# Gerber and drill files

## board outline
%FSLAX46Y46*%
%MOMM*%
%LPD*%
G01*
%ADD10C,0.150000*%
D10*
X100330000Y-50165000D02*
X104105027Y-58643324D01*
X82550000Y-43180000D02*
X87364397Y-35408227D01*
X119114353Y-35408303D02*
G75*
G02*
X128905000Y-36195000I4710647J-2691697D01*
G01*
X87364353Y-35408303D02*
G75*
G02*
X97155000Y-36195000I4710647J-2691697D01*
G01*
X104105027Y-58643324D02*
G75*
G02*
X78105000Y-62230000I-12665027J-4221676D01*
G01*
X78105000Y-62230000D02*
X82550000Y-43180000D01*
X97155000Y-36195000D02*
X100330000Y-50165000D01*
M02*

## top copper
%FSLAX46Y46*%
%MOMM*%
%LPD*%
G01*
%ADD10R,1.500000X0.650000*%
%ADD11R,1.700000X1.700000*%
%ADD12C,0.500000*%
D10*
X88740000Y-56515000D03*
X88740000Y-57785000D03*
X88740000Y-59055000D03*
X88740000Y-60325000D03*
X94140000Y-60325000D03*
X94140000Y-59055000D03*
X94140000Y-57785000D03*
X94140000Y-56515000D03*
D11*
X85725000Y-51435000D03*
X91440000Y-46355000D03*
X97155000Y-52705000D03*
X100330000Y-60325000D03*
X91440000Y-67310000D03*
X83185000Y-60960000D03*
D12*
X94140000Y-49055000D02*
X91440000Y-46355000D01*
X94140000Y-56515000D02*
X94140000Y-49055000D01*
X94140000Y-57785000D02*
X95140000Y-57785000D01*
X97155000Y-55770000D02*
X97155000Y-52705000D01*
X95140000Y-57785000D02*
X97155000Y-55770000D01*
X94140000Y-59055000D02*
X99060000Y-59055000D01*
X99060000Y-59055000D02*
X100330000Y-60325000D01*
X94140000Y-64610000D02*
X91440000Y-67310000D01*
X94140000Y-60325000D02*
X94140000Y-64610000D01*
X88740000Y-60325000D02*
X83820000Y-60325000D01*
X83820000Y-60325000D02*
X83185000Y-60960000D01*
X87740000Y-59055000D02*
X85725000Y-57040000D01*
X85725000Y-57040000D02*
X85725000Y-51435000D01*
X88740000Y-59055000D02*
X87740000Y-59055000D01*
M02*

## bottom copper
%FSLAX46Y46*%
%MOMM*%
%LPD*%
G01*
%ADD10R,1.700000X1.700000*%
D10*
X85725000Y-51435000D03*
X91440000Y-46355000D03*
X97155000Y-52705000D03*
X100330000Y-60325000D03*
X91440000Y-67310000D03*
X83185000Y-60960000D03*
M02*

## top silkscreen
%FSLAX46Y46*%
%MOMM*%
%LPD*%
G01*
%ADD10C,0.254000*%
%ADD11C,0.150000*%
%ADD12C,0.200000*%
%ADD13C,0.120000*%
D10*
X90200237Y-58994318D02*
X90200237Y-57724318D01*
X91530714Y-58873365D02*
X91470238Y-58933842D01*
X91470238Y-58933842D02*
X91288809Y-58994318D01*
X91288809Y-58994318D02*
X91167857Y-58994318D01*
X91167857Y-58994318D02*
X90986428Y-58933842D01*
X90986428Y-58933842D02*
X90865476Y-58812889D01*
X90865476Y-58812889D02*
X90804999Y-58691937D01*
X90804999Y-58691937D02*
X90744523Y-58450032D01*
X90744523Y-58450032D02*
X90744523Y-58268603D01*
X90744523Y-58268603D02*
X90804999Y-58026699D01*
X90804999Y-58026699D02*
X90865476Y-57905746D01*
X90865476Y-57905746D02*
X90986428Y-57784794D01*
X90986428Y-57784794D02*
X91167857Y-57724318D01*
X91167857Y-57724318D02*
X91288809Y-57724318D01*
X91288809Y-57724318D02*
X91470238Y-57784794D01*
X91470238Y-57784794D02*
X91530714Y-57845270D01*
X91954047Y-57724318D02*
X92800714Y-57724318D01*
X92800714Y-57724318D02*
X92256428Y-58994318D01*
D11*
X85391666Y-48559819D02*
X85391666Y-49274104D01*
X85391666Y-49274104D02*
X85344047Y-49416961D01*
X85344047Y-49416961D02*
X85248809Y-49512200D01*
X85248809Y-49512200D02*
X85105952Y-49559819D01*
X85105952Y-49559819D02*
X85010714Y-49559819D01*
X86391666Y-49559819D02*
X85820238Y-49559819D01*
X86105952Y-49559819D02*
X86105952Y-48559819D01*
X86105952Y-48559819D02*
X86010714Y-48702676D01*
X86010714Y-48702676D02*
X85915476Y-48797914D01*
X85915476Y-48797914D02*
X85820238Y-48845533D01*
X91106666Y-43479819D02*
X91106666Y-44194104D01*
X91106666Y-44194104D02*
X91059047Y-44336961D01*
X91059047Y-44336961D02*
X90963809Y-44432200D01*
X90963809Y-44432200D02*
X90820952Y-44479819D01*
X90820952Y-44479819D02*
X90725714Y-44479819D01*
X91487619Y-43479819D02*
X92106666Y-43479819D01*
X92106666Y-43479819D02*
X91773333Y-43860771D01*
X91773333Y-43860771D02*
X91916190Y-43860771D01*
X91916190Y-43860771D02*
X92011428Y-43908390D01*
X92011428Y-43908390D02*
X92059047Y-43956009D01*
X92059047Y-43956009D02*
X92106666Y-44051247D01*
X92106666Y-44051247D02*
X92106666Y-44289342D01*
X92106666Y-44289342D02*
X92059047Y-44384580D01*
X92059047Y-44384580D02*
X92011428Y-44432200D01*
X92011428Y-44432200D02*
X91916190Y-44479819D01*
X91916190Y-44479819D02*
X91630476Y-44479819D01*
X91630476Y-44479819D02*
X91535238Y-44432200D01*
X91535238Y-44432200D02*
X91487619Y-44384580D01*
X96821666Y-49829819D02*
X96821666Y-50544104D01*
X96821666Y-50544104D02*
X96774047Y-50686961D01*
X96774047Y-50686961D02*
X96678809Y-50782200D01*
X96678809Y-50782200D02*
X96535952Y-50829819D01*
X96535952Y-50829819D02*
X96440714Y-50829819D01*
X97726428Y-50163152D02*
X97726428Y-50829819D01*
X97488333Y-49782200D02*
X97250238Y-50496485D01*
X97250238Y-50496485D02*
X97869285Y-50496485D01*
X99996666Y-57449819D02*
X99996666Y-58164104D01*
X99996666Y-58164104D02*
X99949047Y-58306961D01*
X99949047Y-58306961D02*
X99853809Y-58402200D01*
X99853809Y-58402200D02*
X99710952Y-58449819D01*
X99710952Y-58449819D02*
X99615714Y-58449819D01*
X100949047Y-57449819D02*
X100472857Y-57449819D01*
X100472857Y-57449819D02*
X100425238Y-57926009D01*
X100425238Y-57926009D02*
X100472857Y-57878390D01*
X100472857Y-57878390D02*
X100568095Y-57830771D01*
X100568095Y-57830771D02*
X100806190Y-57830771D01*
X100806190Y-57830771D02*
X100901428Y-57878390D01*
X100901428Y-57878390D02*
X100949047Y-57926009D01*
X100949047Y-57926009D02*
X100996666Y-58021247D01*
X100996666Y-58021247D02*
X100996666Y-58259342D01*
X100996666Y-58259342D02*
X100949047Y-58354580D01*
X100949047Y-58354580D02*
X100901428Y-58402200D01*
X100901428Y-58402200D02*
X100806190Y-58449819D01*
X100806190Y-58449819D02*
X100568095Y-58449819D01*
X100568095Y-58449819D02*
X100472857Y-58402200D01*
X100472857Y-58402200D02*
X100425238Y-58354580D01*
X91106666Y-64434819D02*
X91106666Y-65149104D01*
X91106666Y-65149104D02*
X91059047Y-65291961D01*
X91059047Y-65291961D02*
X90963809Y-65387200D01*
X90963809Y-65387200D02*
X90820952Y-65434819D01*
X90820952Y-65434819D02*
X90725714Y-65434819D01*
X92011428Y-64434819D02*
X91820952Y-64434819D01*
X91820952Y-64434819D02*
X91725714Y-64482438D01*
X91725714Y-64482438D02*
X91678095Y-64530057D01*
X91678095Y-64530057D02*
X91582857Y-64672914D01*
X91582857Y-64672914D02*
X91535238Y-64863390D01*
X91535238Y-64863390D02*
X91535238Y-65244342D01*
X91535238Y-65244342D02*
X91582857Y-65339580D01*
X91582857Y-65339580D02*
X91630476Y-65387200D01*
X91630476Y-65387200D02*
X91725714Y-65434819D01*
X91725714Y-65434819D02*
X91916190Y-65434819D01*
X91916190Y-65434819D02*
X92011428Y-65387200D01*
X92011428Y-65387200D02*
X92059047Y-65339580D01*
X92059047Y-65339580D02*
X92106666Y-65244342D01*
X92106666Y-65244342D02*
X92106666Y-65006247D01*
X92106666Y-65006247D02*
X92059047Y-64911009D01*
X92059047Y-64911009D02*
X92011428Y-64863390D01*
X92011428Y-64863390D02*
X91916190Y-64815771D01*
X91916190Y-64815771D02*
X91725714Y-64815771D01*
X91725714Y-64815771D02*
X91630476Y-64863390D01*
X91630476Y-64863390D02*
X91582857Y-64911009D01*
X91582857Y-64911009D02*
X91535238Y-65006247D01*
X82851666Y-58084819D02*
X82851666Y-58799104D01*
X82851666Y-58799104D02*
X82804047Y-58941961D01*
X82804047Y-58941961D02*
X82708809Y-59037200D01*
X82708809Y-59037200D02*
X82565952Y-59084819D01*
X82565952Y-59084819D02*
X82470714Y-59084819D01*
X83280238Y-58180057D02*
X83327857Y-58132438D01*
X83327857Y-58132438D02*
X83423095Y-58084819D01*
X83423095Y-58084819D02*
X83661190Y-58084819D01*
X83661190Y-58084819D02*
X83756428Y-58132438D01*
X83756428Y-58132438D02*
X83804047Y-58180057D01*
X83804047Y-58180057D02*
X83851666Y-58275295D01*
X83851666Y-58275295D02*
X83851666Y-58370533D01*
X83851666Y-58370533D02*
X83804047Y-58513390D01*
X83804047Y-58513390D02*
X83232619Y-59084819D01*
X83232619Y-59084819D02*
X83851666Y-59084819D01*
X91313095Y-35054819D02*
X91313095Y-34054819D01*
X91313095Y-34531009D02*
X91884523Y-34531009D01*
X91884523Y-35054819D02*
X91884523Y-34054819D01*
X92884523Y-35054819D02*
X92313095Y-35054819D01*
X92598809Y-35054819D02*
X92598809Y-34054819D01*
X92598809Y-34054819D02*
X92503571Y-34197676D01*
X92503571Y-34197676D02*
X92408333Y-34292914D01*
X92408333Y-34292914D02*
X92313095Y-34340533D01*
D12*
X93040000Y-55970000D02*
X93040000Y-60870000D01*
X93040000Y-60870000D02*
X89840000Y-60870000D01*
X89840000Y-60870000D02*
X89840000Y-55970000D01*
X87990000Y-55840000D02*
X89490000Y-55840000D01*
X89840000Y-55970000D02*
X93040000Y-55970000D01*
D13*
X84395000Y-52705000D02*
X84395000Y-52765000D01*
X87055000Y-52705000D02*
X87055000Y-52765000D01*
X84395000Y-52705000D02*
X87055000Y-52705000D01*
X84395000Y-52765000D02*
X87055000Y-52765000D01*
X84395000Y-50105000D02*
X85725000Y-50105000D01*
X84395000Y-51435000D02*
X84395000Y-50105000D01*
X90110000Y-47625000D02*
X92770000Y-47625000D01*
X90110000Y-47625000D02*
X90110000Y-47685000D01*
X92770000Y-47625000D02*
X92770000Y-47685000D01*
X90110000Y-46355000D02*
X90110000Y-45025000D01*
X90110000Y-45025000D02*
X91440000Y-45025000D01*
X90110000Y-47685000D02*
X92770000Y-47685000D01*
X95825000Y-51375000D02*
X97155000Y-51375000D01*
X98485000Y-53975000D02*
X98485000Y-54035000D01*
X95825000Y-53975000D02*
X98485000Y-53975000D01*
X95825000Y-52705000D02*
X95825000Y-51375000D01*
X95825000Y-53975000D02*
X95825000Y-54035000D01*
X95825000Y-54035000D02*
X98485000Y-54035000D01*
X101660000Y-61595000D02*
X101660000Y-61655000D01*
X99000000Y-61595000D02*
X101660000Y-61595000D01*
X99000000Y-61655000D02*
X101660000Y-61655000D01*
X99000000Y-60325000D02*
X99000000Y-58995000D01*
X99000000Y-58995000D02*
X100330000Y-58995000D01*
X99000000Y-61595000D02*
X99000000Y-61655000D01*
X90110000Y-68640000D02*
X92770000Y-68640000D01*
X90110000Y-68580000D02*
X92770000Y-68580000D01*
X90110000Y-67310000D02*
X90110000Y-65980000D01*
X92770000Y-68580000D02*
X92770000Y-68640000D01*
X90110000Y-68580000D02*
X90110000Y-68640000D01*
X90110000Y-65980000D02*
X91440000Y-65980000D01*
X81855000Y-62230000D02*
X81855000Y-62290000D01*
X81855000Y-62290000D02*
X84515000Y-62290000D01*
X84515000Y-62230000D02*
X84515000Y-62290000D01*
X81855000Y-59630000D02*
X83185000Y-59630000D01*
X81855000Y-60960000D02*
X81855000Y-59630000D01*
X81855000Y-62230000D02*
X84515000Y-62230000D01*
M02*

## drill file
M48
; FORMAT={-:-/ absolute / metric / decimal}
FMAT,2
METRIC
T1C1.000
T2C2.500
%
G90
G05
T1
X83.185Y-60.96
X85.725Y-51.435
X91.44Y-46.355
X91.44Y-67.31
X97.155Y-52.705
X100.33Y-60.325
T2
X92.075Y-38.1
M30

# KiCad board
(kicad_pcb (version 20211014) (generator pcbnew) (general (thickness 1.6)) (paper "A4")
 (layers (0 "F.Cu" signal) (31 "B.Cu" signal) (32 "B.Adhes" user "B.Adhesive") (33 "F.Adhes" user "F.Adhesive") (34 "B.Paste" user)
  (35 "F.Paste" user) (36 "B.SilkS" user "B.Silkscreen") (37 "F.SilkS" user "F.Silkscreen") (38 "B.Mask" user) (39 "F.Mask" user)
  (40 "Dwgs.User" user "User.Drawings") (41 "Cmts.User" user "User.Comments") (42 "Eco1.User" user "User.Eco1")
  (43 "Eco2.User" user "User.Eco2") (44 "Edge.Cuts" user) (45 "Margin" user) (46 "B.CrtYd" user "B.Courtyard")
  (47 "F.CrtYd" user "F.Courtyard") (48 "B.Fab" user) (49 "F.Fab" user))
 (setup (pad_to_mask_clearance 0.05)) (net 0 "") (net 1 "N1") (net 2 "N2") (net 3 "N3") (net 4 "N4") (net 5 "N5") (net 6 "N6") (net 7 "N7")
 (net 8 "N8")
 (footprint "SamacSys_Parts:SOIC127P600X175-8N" (layer "F.Cu") (at 91.44 58.42)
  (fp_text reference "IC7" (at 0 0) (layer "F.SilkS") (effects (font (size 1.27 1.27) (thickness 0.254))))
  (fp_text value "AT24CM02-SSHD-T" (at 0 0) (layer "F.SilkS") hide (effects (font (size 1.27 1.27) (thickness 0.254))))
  (fp_line (start 1.6 -2.45) (end 1.6 2.45) (layer "F.SilkS") (width 0.2))
  (fp_line (start 1.6 2.45) (end -1.6 2.45) (layer "F.SilkS") (width 0.2))
  (fp_line (start -1.6 2.45) (end -1.6 -2.45) (layer "F.SilkS") (width 0.2))
  (fp_line (start -3.45 -2.58) (end -1.95 -2.58) (layer "F.SilkS") (width 0.2))
  (fp_line (start -1.6 -2.45) (end 1.6 -2.45) (layer "F.SilkS") (width 0.2))
  (pad "1" smd rect locked (at -2.7 -1.905 90) (size 0.65 1.5) (layers "F.Cu" "F.Paste" "F.Mask") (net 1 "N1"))
  (pad "2" smd rect locked (at -2.7 -0.635 90) (size 0.65 1.5) (layers "F.Cu" "F.Paste" "F.Mask") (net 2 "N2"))
  (pad "3" smd rect locked (at -2.7 0.635 90) (size 0.65 1.5) (layers "F.Cu" "F.Paste" "F.Mask") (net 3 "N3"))
  (pad "4" smd rect locked (at -2.7 1.905 90) (size 0.65 1.5) (layers "F.Cu" "F.Paste" "F.Mask") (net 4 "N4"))
  (pad "5" smd rect locked (at 2.7 1.905 90) (size 0.65 1.5) (layers "F.Cu" "F.Paste" "F.Mask") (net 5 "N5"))
  (pad "6" smd rect locked (at 2.7 0.635 90) (size 0.65 1.5) (layers "F.Cu" "F.Paste" "F.Mask") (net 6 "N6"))
  (pad "7" smd rect locked (at 2.7 -0.635 90) (size 0.65 1.5) (layers "F.Cu" "F.Paste" "F.Mask") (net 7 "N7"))
  (pad "8" smd rect locked (at 2.7 -1.905 90) (size 0.65 1.5) (layers "F.Cu" "F.Paste" "F.Mask") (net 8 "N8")))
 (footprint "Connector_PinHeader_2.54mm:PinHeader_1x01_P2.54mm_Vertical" (layer "F.Cu") (at 85.725 51.435)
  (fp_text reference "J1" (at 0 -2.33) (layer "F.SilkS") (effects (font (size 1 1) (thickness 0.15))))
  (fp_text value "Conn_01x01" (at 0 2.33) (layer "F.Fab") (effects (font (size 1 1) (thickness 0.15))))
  (fp_line (start -1.33 1.27) (end -1.33 1.33) (layer "F.SilkS") (width 0.12))
  (fp_line (start 1.33 1.27) (end 1.33 1.33) (layer "F.SilkS") (width 0.12))
  (fp_line (start -1.33 1.27) (end 1.33 1.27) (layer "F.SilkS") (width 0.12))
  (fp_line (start -1.33 1.33) (end 1.33 1.33) (layer "F.SilkS") (width 0.12))
  (fp_line (start -1.33 -1.33) (end 0 -1.33) (layer "F.SilkS") (width 0.12))
  (fp_line (start -1.33 0) (end -1.33 -1.33) (layer "F.SilkS") (width 0.12))
  (pad "1" thru_hole rect locked (at 0 0) (size 1.7 1.7) (drill 1) (layers *.Cu *.Mask) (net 3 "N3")))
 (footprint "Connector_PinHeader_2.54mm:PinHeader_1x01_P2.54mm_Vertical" (layer "F.Cu") (at 91.44 46.355)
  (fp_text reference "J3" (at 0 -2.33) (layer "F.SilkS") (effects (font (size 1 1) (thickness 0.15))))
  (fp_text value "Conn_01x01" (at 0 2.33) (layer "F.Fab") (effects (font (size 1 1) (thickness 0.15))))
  (fp_line (start -1.33 1.27) (end 1.33 1.27) (layer "F.SilkS") (width 0.12))
  (fp_line (start -1.33 1.27) (end -1.33 1.33) (layer "F.SilkS") (width 0.12))
  (fp_line (start 1.33 1.27) (end 1.33 1.33) (layer "F.SilkS") (width 0.12))
  (fp_line (start -1.33 0) (end -1.33 -1.33) (layer "F.SilkS") (width 0.12))
  (fp_line (start -1.33 -1.33) (end 0 -1.33) (layer "F.SilkS") (width 0.12))
  (fp_line (start -1.33 1.33) (end 1.33 1.33) (layer "F.SilkS") (width 0.12))
  (pad "1" thru_hole rect locked (at 0 0) (size 1.7 1.7) (drill 1) (layers *.Cu *.Mask) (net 8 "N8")))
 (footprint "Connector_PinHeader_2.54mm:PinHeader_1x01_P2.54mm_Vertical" (layer "F.Cu") (at 97.155 52.705)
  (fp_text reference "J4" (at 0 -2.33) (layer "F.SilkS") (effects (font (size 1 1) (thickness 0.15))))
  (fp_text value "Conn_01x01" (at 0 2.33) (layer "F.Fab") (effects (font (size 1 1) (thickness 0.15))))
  (fp_line (start -1.33 -1.33) (end 0 -1.33) (layer "F.SilkS") (width 0.12))
  (fp_line (start 1.33 1.27) (end 1.33 1.33) (layer "F.SilkS") (width 0.12))
  (fp_line (start -1.33 1.27) (end 1.33 1.27) (layer "F.SilkS") (width 0.12))
  (fp_line (start -1.33 0) (end -1.33 -1.33) (layer "F.SilkS") (width 0.12))
  (fp_line (start -1.33 1.27) (end -1.33 1.33) (layer "F.SilkS") (width 0.12))
  (fp_line (start -1.33 1.33) (end 1.33 1.33) (layer "F.SilkS") (width 0.12))
  (pad "1" thru_hole rect locked (at 0 0) (size 1.7 1.7) (drill 1) (layers *.Cu *.Mask) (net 7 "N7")))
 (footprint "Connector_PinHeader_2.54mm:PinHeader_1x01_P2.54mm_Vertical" (layer "F.Cu") (at 100.33 60.325)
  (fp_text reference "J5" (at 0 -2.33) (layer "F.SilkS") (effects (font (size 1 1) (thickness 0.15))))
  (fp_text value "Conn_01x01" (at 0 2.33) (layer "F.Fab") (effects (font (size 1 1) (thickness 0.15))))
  (fp_line (start 1.33 1.27) (end 1.33 1.33) (layer "F.SilkS") (width 0.12))
  (fp_line (start -1.33 1.27) (end 1.33 1.27) (layer "F.SilkS") (width 0.12))
  (fp_line (start -1.33 1.33) (end 1.33 1.33) (layer "F.SilkS") (width 0.12))
  (fp_line (start -1.33 0) (end -1.33 -1.33) (layer "F.SilkS") (width 0.12))
  (fp_line (start -1.33 -1.33) (end 0 -1.33) (layer "F.SilkS") (width 0.12))
  (fp_line (start -1.33 1.27) (end -1.33 1.33) (layer "F.SilkS") (width 0.12))
  (pad "1" thru_hole rect locked (at 0 0) (size 1.7 1.7) (drill 1) (layers *.Cu *.Mask) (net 6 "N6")))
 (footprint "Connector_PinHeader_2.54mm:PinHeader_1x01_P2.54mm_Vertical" (layer "F.Cu") (at 91.44 67.31)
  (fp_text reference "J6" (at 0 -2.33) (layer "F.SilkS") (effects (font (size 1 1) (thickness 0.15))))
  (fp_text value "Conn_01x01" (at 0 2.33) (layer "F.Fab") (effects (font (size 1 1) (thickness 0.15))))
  (fp_line (start -1.33 1.33) (end 1.33 1.33) (layer "F.SilkS") (width 0.12))
  (fp_line (start -1.33 1.27) (end 1.33 1.27) (layer "F.SilkS") (width 0.12))
  (fp_line (start -1.33 0) (end -1.33 -1.33) (layer "F.SilkS") (width 0.12))
  (fp_line (start 1.33 1.27) (end 1.33 1.33) (layer "F.SilkS") (width 0.12))
  (fp_line (start -1.33 1.27) (end -1.33 1.33) (layer "F.SilkS") (width 0.12))
  (fp_line (start -1.33 -1.33) (end 0 -1.33) (layer "F.SilkS") (width 0.12))
  (pad "1" thru_hole rect locked (at 0 0) (size 1.7 1.7) (drill 1) (layers *.Cu *.Mask) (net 5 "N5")))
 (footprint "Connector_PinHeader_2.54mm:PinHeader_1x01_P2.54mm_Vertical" (layer "F.Cu") (at 83.185 60.96)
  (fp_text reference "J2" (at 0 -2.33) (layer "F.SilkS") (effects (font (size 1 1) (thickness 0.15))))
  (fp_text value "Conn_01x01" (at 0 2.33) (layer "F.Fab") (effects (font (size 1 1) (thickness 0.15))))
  (fp_line (start -1.33 1.27) (end -1.33 1.33) (layer "F.SilkS") (width 0.12))
  (fp_line (start -1.33 1.33) (end 1.33 1.33) (layer "F.SilkS") (width 0.12))
  (fp_line (start 1.33 1.27) (end 1.33 1.33) (layer "F.SilkS") (width 0.12))
  (fp_line (start -1.33 -1.33) (end 0 -1.33) (layer "F.SilkS") (width 0.12))
  (fp_line (start -1.33 0) (end -1.33 -1.33) (layer "F.SilkS") (width 0.12))
  (fp_line (start -1.33 1.27) (end 1.33 1.27) (layer "F.SilkS") (width 0.12))
  (pad "1" thru_hole rect locked (at 0 0) (size 1.7 1.7) (drill 1) (layers *.Cu *.Mask) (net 4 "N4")))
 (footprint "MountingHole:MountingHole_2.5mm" (layer "F.Cu") (at 92.075 38.1)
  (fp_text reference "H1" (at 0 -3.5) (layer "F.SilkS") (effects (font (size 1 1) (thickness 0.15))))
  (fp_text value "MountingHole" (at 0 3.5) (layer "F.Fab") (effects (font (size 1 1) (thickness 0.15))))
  (pad "" np_thru_hole circle locked (at 0 0) (size 2.5 2.5) (drill 2.5) (layers *.Cu *.Mask)))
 (gr_line (start 100.33 50.165) (end 104.105027 58.643324) (layer "Edge.Cuts") (width 0.15))
 (gr_line (start 82.55 43.18) (end 87.364397 35.408227) (layer "Edge.Cuts") (width 0.15))
 (gr_arc (start 119.114353 35.408303) (mid 124.259544 32.691987) (end 128.905 36.195) (layer "Edge.Cuts") (width 0.15))
 (gr_arc (start 87.364353 35.408303) (mid 92.509544 32.691987) (end 97.155 36.195) (layer "Edge.Cuts") (width 0.15))
 (gr_arc (start 104.105027 58.643324) (mid 93.264357 76.08987) (end 78.105 62.23) (layer "Edge.Cuts") (width 0.15))
 (gr_line (start 78.105 62.23) (end 82.55 43.18) (layer "Edge.Cuts") (width 0.15))
 (gr_line (start 97.155 36.195) (end 100.33 50.165) (layer "Edge.Cuts") (width 0.15))
 (segment (start 94.14 49.055) (end 91.44 46.355) (width 0.5) (layer "F.Cu") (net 8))
 (segment (start 94.14 56.515) (end 94.14 49.055) (width 0.5) (layer "F.Cu") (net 8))
 (segment (start 94.14 57.785) (end 95.14 57.785) (width 0.5) (layer "F.Cu") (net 7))
 (segment (start 97.155 55.77) (end 97.155 52.705) (width 0.5) (layer "F.Cu") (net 7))
 (segment (start 95.14 57.785) (end 97.155 55.77) (width 0.5) (layer "F.Cu") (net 7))
 (segment (start 94.14 59.055) (end 99.06 59.055) (width 0.5) (layer "F.Cu") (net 6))
 (segment (start 99.06 59.055) (end 100.33 60.325) (width 0.5) (layer "F.Cu") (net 6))
 (segment (start 94.14 64.61) (end 91.44 67.31) (width 0.5) (layer "F.Cu") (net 5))
 (segment (start 94.14 60.325) (end 94.14 64.61) (width 0.5) (layer "F.Cu") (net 5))
 (segment (start 88.74 60.325) (end 83.82 60.325) (width 0.5) (layer "F.Cu") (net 4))
 (segment (start 83.82 60.325) (end 83.185 60.96) (width 0.5) (layer "F.Cu") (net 4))
 (segment (start 87.74 59.055) (end 85.725 57.04) (width 0.5) (layer "F.Cu") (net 3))
 (segment (start 85.725 57.04) (end 85.725 51.435) (width 0.5) (layer "F.Cu") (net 3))
 (segment (start 88.74 59.055) (end 87.74 59.055) (width 0.5) (layer "F.Cu") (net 3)))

